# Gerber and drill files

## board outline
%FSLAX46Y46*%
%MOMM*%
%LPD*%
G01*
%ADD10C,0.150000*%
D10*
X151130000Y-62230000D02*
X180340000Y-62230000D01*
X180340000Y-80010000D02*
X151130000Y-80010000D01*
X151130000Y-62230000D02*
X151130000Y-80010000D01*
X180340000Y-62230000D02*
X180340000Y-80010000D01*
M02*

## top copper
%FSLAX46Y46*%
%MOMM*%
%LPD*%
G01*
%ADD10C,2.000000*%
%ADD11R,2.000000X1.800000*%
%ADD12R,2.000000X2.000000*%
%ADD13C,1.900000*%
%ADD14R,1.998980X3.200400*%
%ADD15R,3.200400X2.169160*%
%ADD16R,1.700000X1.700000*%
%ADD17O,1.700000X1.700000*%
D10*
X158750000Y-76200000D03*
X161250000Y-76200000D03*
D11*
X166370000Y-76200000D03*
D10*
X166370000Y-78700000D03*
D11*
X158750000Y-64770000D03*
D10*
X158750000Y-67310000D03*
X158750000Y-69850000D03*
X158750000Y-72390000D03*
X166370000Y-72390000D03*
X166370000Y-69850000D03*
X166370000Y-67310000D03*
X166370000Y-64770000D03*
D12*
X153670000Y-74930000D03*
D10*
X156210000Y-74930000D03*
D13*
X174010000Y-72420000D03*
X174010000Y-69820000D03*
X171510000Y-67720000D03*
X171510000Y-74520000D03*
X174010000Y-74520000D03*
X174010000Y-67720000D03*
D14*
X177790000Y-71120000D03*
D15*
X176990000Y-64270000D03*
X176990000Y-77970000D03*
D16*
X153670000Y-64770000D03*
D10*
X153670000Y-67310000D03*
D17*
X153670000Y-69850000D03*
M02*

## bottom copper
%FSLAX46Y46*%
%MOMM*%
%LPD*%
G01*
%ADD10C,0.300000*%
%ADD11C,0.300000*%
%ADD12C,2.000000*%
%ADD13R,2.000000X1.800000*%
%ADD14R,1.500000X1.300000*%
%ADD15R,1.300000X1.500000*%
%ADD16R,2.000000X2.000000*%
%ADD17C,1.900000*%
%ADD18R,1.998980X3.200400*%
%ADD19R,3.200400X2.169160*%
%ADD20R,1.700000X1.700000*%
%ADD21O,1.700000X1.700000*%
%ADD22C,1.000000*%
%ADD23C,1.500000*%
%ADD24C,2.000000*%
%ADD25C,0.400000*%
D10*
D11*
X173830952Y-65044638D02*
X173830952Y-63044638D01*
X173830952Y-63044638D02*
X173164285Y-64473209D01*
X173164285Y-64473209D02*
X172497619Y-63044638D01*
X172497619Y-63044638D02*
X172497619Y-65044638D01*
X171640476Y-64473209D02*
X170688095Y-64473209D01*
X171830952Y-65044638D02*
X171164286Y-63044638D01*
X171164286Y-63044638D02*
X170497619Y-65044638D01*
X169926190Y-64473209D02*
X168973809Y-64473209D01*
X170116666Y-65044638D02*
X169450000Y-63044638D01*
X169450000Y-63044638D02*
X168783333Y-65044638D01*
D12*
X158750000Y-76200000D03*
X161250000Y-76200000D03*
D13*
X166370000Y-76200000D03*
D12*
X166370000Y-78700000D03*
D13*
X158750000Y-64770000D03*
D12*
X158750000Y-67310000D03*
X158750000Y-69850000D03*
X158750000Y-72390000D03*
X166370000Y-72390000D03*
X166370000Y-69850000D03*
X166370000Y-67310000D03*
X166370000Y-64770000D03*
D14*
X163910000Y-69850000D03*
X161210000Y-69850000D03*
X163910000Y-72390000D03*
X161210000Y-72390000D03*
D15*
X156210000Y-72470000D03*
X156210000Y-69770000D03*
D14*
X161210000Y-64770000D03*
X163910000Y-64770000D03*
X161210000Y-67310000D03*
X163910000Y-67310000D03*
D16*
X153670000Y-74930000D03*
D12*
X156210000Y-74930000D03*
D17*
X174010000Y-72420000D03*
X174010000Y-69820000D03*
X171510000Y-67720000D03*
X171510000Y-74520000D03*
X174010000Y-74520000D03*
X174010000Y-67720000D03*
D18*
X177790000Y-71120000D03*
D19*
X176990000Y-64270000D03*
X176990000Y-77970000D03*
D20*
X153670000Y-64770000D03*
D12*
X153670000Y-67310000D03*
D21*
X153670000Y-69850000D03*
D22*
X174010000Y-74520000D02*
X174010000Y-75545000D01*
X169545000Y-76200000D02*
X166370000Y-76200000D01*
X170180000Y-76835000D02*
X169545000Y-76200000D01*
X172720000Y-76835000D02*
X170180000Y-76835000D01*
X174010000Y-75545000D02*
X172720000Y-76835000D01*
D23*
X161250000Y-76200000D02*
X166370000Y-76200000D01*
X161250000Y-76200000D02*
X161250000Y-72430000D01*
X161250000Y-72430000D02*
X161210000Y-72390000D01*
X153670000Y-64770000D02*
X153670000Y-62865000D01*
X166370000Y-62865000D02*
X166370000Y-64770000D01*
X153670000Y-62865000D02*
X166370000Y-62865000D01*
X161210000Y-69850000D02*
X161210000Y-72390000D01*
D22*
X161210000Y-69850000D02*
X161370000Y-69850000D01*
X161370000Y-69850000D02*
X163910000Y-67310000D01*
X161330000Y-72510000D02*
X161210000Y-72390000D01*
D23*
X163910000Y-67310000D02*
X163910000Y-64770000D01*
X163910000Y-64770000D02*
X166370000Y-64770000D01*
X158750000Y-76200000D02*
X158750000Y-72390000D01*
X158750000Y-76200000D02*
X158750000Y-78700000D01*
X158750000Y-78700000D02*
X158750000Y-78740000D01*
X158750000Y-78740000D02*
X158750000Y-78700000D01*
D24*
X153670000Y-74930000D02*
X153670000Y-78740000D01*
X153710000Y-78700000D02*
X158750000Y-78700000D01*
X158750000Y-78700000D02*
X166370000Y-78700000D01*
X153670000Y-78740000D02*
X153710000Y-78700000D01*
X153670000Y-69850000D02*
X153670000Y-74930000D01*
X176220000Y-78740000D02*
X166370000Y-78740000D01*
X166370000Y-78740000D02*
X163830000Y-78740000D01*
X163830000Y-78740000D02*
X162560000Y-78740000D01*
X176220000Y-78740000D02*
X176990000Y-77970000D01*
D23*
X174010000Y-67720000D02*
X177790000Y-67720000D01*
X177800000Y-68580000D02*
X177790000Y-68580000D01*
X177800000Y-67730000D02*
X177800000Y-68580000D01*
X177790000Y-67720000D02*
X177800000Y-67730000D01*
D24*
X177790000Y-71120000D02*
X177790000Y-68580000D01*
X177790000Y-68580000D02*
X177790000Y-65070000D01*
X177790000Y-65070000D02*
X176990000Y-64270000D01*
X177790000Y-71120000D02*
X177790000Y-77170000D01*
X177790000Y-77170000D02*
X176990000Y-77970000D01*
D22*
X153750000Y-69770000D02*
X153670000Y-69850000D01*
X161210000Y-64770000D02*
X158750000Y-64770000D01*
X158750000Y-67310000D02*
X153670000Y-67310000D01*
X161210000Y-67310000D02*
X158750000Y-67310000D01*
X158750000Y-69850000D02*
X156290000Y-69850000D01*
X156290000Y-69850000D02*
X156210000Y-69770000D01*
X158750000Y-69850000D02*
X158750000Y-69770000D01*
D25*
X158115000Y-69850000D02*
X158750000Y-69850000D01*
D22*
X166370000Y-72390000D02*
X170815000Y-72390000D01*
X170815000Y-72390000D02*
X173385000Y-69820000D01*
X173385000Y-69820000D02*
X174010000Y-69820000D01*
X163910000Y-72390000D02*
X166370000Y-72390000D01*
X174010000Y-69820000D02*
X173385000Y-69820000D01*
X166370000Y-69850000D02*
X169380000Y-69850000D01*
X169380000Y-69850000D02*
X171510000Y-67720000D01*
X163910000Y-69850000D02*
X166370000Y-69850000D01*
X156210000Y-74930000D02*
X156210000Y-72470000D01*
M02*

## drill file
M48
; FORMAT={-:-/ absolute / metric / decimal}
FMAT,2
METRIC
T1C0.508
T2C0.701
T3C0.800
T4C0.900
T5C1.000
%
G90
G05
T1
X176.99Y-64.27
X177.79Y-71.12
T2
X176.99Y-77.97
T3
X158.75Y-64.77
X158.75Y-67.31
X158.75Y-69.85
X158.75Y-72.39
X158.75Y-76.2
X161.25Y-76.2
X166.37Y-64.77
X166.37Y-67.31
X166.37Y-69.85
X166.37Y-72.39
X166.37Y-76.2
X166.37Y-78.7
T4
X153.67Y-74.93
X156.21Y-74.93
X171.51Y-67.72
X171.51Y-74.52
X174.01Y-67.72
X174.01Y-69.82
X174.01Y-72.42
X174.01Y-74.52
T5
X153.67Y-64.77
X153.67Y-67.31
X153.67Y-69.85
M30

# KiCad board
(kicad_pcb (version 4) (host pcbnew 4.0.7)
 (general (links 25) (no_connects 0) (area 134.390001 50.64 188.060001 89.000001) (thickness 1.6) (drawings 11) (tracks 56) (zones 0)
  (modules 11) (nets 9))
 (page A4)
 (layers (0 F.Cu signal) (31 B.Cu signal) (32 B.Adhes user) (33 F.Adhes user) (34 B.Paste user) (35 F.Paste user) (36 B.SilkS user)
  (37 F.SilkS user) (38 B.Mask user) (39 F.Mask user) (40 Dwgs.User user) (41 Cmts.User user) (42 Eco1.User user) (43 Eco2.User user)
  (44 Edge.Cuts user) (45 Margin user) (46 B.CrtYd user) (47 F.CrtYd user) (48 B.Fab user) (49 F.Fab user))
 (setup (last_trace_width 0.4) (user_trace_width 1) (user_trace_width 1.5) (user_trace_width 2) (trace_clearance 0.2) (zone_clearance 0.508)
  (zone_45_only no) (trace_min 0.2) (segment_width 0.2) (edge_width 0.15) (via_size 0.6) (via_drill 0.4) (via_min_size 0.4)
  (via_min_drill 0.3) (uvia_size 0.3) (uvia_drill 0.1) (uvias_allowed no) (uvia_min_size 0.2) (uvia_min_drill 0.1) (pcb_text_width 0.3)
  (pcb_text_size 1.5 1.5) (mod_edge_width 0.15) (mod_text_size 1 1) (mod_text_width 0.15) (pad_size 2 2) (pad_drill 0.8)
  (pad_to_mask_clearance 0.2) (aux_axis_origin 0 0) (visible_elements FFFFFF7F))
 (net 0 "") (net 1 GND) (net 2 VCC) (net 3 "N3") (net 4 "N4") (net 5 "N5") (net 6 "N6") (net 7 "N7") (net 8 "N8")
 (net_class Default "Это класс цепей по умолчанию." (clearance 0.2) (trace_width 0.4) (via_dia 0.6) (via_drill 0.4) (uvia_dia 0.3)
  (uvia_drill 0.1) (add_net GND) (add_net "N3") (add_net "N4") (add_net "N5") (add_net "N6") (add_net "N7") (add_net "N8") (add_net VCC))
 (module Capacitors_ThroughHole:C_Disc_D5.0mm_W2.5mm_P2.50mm (layer F.Cu) (at 158.75 76.2)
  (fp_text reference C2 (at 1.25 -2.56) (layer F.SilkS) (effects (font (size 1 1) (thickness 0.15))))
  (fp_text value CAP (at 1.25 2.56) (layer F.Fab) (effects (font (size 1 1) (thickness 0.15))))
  (pad 1 thru_hole circle (at 0 0) (size 2 2) (drill 0.8) (layers *.Cu *.Mask) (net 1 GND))
  (pad 2 thru_hole circle (at 2.5 0) (size 2 2) (drill 0.8) (layers *.Cu *.Mask) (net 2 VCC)))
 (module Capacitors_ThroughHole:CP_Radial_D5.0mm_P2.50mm (layer F.Cu) (at 166.37 76.2 270)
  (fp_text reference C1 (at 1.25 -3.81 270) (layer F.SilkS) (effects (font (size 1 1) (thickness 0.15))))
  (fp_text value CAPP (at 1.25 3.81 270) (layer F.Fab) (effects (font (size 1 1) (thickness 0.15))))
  (pad 1 thru_hole rect (at 0 0 270) (size 1.8 2) (drill 0.8) (layers *.Cu *.Mask) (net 2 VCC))
  (pad 2 thru_hole circle (at 2.5 0 270) (size 2 2) (drill 0.8) (layers *.Cu *.Mask) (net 1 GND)))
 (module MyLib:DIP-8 (layer F.Cu) (at 158.75 64.77 270)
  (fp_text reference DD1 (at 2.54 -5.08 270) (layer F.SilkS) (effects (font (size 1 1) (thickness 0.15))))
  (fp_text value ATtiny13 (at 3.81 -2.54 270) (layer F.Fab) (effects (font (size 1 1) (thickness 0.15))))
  (pad 1 thru_hole rect (at 0 0 270) (size 1.8 2) (drill 0.8) (layers *.Cu *.Mask F.SilkS) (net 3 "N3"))
  (pad 2 thru_hole circle (at 2.54 0 270) (size 2 2) (drill 0.8) (layers *.Cu *.Mask F.SilkS) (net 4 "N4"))
  (pad 3 thru_hole circle (at 5.08 0 270) (size 2 2) (drill 0.8) (layers *.Cu *.Mask F.SilkS) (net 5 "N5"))
  (pad 4 thru_hole circle (at 7.62 0 270) (size 2 2) (drill 0.8) (layers *.Cu *.Mask F.SilkS) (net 1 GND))
  (pad 5 thru_hole circle (at 7.62 -7.62 270) (size 2 2) (drill 0.8) (layers *.Cu *.Mask F.SilkS) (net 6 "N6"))
  (pad 6 thru_hole circle (at 5.08 -7.62 270) (size 2 2) (drill 0.8) (layers *.Cu *.Mask F.SilkS) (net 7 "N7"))
  (pad 7 thru_hole circle (at 2.54 -7.62 270) (size 2 2) (drill 0.8) (layers *.Cu *.Mask F.SilkS))
  (pad 8 thru_hole circle (at 0 -7.62 270) (size 2 2) (drill 0.8) (layers *.Cu *.Mask F.SilkS) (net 2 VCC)))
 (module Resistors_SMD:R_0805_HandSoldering (layer B.Cu) (at 162.56 69.85 180)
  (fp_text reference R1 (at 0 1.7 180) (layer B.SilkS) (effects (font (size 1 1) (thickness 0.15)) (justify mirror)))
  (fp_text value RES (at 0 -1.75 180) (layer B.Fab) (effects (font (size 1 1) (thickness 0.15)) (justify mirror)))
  (pad 1 smd rect (at -1.35 0 180) (size 1.5 1.3) (layers B.Cu B.Paste B.Mask) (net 7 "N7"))
  (pad 2 smd rect (at 1.35 0 180) (size 1.5 1.3) (layers B.Cu B.Paste B.Mask) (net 2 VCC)))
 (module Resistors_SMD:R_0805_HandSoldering (layer B.Cu) (at 162.56 72.39 180)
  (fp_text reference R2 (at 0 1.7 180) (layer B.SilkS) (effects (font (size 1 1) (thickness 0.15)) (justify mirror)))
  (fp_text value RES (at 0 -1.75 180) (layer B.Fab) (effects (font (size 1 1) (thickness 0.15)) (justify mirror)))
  (pad 1 smd rect (at -1.35 0 180) (size 1.5 1.3) (layers B.Cu B.Paste B.Mask) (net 6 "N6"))
  (pad 2 smd rect (at 1.35 0 180) (size 1.5 1.3) (layers B.Cu B.Paste B.Mask) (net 2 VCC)))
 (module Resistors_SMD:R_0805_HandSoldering (layer B.Cu) (at 156.21 71.12 90)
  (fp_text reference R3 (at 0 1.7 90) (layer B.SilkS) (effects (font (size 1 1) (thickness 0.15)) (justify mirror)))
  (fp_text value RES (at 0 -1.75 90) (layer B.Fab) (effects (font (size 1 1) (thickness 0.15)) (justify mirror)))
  (pad 1 smd rect (at -1.35 0 90) (size 1.5 1.3) (layers B.Cu B.Paste B.Mask) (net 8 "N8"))
  (pad 2 smd rect (at 1.35 0 90) (size 1.5 1.3) (layers B.Cu B.Paste B.Mask) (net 5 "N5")))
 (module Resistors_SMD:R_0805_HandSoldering (layer B.Cu) (at 162.56 64.77)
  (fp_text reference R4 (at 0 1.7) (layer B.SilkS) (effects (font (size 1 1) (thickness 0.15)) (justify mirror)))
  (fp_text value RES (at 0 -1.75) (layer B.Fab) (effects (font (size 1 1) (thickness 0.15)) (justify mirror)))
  (pad 1 smd rect (at -1.35 0) (size 1.5 1.3) (layers B.Cu B.Paste B.Mask) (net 3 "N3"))
  (pad 2 smd rect (at 1.35 0) (size 1.5 1.3) (layers B.Cu B.Paste B.Mask) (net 2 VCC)))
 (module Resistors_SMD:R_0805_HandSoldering (layer B.Cu) (at 162.56 67.31)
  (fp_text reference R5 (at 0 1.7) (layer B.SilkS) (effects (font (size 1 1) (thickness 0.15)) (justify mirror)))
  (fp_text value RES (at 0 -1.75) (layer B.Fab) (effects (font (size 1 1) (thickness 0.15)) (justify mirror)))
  (pad 1 smd rect (at -1.35 0) (size 1.5 1.3) (layers B.Cu B.Paste B.Mask) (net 4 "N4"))
  (pad 2 smd rect (at 1.35 0) (size 1.5 1.3) (layers B.Cu B.Paste B.Mask) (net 2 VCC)))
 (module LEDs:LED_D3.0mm (layer F.Cu) (at 153.67 74.93)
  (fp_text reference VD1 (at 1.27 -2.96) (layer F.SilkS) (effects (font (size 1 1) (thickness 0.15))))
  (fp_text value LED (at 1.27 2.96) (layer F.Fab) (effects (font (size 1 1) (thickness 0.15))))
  (pad 1 thru_hole rect (at 0 0) (size 2 2) (drill 0.9) (layers *.Cu *.Mask) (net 1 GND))
  (pad 2 thru_hole circle (at 2.54 0) (size 2 2) (drill 0.9) (layers *.Cu *.Mask) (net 8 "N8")))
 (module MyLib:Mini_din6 (layer F.Cu) (at 175.26 71.12 90)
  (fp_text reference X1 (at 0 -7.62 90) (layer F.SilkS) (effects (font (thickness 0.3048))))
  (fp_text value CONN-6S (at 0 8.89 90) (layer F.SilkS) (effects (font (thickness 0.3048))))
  (pad 2 thru_hole circle (at -1.3 -1.25 90) (size 1.9 1.9) (drill 0.9) (layers *.Cu *.Mask F.SilkS))
  (pad 1 thru_hole circle (at 1.3 -1.25 90) (size 1.9 1.9) (drill 0.9) (layers *.Cu *.Mask F.SilkS) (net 6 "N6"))
  (pad 5 thru_hole circle (at 3.4 -3.75 90) (size 1.9 1.9) (drill 0.9) (layers *.Cu *.Mask F.SilkS) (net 7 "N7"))
  (pad 6 thru_hole circle (at -3.4 -3.75 90) (size 1.9 1.9) (drill 0.9) (layers *.Cu *.Mask F.SilkS))
  (pad 4 thru_hole circle (at -3.4 -1.25 90) (size 1.9 1.9) (drill 0.9) (layers *.Cu *.Mask F.SilkS) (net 2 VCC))
  (pad 3 thru_hole circle (at 3.4 -1.25 90) (size 1.9 1.9) (drill 0.9) (layers *.Cu *.Mask F.SilkS) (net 1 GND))
  (pad S thru_hole rect (at 0 2.53 90) (size 3.2004 1.99898) (drill 0.508) (layers *.Cu *.SilkS *.Mask) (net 1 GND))
  (pad S thru_hole rect (at 6.85 1.73 90) (size 2.16916 3.2004) (drill 0.508) (layers *.Cu *.SilkS *.Mask) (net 1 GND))
  (pad S thru_hole rect (at -6.85 1.73 90) (size 2.16916 3.2004) (drill 0.70104) (layers *.Cu *.SilkS *.Mask) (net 1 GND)))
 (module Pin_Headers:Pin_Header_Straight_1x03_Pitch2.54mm (layer F.Cu) (at 153.67 64.77)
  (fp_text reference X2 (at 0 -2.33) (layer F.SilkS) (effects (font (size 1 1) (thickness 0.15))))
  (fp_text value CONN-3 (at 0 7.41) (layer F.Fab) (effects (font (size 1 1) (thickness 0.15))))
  (pad 1 thru_hole rect (at 0 0) (size 1.7 1.7) (drill 1) (layers *.Cu *.Mask) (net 2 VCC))
  (pad 2 thru_hole circle (at 0 2.54) (size 2 2) (drill 1) (layers *.Cu *.Mask) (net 4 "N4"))
  (pad 3 thru_hole oval (at 0 5.08) (size 1.7 1.7) (drill 1) (layers *.Cu *.Mask) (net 1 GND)))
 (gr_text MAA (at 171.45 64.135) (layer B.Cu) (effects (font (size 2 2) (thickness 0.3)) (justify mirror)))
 (gr_line (start 151.13 62.23) (end 180.34 62.23) (angle 90) (layer Edge.Cuts) (width 0.15))
 (gr_line (start 180.34 80.01) (end 151.13 80.01) (angle 90) (layer Edge.Cuts) (width 0.15))
 (gr_line (start 151.13 62.23) (end 151.13 80.01) (angle 90) (layer Edge.Cuts) (width 0.15))
 (gr_line (start 180.34 62.23) (end 180.34 80.01) (angle 90) (layer Edge.Cuts) (width 0.15))
 (segment (start 174.01 74.52) (end 174.01 75.545) (width 1) (layer B.Cu) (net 2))
 (segment (start 169.545 76.2) (end 166.37 76.2) (width 1) (layer B.Cu) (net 2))
 (segment (start 170.18 76.835) (end 169.545 76.2) (width 1) (layer B.Cu) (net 2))
 (segment (start 172.72 76.835) (end 170.18 76.835) (width 1) (layer B.Cu) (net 2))
 (segment (start 174.01 75.545) (end 172.72 76.835) (width 1) (layer B.Cu) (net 2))
 (segment (start 161.25 76.2) (end 166.37 76.2) (width 1.5) (layer B.Cu) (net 2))
 (segment (start 161.25 76.2) (end 161.25 72.43) (width 1.5) (layer B.Cu) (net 2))
 (segment (start 161.25 72.43) (end 161.21 72.39) (width 1.5) (layer B.Cu) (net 2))
 (segment (start 153.67 64.77) (end 153.67 62.865) (width 1.5) (layer B.Cu) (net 2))
 (segment (start 166.37 62.865) (end 166.37 64.77) (width 1.5) (layer B.Cu) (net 2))
 (segment (start 153.67 62.865) (end 166.37 62.865) (width 1.5) (layer B.Cu) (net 2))
 (segment (start 161.21 69.85) (end 161.21 72.39) (width 1.5) (layer B.Cu) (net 2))
 (segment (start 161.21 69.85) (end 161.37 69.85) (width 1) (layer B.Cu) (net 2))
 (segment (start 161.37 69.85) (end 163.91 67.31) (width 1) (layer B.Cu) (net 2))
 (segment (start 161.33 72.51) (end 161.21 72.39) (width 1) (layer B.Cu) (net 2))
 (segment (start 163.91 67.31) (end 163.91 64.77) (width 1.5) (layer B.Cu) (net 2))
 (segment (start 163.91 64.77) (end 166.37 64.77) (width 1.5) (layer B.Cu) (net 2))
 (segment (start 158.75 76.2) (end 158.75 72.39) (width 1.5) (layer B.Cu) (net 1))
 (segment (start 158.75 76.2) (end 158.75 78.7) (width 1.5) (layer B.Cu) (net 1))
 (segment (start 158.75 78.7) (end 158.75 78.74) (width 1.5) (layer B.Cu) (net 1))
 (segment (start 158.75 78.74) (end 158.75 78.7) (width 1.5) (layer B.Cu) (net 1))
 (segment (start 153.67 74.93) (end 153.67 78.74) (width 2) (layer B.Cu) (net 1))
 (segment (start 153.71 78.7) (end 158.75 78.7) (width 2) (layer B.Cu) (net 1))
 (segment (start 158.75 78.7) (end 166.37 78.7) (width 2) (layer B.Cu) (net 1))
 (segment (start 153.67 78.74) (end 153.71 78.7) (width 2) (layer B.Cu) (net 1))
 (segment (start 153.67 69.85) (end 153.67 74.93) (width 2) (layer B.Cu) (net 1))
 (segment (start 176.22 78.74) (end 166.37 78.74) (width 2) (layer B.Cu) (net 1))
 (segment (start 166.37 78.74) (end 163.83 78.74) (width 2) (layer B.Cu) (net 1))
 (segment (start 163.83 78.74) (end 162.56 78.74) (width 2) (layer B.Cu) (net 1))
 (segment (start 176.22 78.74) (end 176.99 77.97) (width 2) (layer B.Cu) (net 1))
 (segment (start 174.01 67.72) (end 177.79 67.72) (width 1.5) (layer B.Cu) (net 1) (status 10))
 (segment (start 177.8 68.58) (end 177.79 68.58) (width 1.5) (layer B.Cu) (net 1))
 (segment (start 177.8 67.73) (end 177.8 68.58) (width 1.5) (layer B.Cu) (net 1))
 (segment (start 177.79 67.72) (end 177.8 67.73) (width 1.5) (layer B.Cu) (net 1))
 (segment (start 177.79 71.12) (end 177.79 68.58) (width 2) (layer B.Cu) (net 1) (status 10))
 (segment (start 177.79 68.58) (end 177.79 65.07) (width 2) (layer B.Cu) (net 1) (status 20))
 (segment (start 177.79 65.07) (end 176.99 64.27) (width 2) (layer B.Cu) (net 1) (status 30))
 (segment (start 177.79 71.12) (end 177.79 77.17) (width 2) (layer B.Cu) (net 1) (status 30))
 (segment (start 177.79 77.17) (end 176.99 77.97) (width 2) (layer B.Cu) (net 1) (status 30))
 (segment (start 153.75 69.77) (end 153.67 69.85) (width 1) (layer B.Cu) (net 1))
 (segment (start 161.21 64.77) (end 158.75 64.77) (width 1) (layer B.Cu) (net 3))
 (segment (start 158.75 67.31) (end 153.67 67.31) (width 1) (layer B.Cu) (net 4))
 (segment (start 161.21 67.31) (end 158.75 67.31) (width 1) (layer B.Cu) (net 4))
 (segment (start 158.75 69.85) (end 156.29 69.85) (width 1) (layer B.Cu) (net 5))
 (segment (start 156.29 69.85) (end 156.21 69.77) (width 1) (layer B.Cu) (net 5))
 (segment (start 158.75 69.85) (end 158.75 69.77) (width 1) (layer B.Cu) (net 5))
 (segment (start 158.115 69.85) (end 158.75 69.85) (width 0.4) (layer B.Cu) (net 5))
 (segment (start 166.37 72.39) (end 170.815 72.39) (width 1) (layer B.Cu) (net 6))
 (segment (start 170.815 72.39) (end 173.385 69.82) (width 1) (layer B.Cu) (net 6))
 (segment (start 173.385 69.82) (end 174.01 69.82) (width 1) (layer B.Cu) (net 6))
 (segment (start 163.91 72.39) (end 166.37 72.39) (width 1) (layer B.Cu) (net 6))
 (segment (start 174.01 69.82) (end 173.385 69.82) (width 1) (layer B.Cu) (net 6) (status 30))
 (segment (start 166.37 69.85) (end 169.38 69.85) (width 1) (layer B.Cu) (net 7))
 (segment (start 169.38 69.85) (end 171.51 67.72) (width 1) (layer B.Cu) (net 7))
 (segment (start 163.91 69.85) (end 166.37 69.85) (width 1) (layer B.Cu) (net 7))
 (segment (start 156.21 74.93) (end 156.21 72.47) (width 1) (layer B.Cu) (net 8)))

